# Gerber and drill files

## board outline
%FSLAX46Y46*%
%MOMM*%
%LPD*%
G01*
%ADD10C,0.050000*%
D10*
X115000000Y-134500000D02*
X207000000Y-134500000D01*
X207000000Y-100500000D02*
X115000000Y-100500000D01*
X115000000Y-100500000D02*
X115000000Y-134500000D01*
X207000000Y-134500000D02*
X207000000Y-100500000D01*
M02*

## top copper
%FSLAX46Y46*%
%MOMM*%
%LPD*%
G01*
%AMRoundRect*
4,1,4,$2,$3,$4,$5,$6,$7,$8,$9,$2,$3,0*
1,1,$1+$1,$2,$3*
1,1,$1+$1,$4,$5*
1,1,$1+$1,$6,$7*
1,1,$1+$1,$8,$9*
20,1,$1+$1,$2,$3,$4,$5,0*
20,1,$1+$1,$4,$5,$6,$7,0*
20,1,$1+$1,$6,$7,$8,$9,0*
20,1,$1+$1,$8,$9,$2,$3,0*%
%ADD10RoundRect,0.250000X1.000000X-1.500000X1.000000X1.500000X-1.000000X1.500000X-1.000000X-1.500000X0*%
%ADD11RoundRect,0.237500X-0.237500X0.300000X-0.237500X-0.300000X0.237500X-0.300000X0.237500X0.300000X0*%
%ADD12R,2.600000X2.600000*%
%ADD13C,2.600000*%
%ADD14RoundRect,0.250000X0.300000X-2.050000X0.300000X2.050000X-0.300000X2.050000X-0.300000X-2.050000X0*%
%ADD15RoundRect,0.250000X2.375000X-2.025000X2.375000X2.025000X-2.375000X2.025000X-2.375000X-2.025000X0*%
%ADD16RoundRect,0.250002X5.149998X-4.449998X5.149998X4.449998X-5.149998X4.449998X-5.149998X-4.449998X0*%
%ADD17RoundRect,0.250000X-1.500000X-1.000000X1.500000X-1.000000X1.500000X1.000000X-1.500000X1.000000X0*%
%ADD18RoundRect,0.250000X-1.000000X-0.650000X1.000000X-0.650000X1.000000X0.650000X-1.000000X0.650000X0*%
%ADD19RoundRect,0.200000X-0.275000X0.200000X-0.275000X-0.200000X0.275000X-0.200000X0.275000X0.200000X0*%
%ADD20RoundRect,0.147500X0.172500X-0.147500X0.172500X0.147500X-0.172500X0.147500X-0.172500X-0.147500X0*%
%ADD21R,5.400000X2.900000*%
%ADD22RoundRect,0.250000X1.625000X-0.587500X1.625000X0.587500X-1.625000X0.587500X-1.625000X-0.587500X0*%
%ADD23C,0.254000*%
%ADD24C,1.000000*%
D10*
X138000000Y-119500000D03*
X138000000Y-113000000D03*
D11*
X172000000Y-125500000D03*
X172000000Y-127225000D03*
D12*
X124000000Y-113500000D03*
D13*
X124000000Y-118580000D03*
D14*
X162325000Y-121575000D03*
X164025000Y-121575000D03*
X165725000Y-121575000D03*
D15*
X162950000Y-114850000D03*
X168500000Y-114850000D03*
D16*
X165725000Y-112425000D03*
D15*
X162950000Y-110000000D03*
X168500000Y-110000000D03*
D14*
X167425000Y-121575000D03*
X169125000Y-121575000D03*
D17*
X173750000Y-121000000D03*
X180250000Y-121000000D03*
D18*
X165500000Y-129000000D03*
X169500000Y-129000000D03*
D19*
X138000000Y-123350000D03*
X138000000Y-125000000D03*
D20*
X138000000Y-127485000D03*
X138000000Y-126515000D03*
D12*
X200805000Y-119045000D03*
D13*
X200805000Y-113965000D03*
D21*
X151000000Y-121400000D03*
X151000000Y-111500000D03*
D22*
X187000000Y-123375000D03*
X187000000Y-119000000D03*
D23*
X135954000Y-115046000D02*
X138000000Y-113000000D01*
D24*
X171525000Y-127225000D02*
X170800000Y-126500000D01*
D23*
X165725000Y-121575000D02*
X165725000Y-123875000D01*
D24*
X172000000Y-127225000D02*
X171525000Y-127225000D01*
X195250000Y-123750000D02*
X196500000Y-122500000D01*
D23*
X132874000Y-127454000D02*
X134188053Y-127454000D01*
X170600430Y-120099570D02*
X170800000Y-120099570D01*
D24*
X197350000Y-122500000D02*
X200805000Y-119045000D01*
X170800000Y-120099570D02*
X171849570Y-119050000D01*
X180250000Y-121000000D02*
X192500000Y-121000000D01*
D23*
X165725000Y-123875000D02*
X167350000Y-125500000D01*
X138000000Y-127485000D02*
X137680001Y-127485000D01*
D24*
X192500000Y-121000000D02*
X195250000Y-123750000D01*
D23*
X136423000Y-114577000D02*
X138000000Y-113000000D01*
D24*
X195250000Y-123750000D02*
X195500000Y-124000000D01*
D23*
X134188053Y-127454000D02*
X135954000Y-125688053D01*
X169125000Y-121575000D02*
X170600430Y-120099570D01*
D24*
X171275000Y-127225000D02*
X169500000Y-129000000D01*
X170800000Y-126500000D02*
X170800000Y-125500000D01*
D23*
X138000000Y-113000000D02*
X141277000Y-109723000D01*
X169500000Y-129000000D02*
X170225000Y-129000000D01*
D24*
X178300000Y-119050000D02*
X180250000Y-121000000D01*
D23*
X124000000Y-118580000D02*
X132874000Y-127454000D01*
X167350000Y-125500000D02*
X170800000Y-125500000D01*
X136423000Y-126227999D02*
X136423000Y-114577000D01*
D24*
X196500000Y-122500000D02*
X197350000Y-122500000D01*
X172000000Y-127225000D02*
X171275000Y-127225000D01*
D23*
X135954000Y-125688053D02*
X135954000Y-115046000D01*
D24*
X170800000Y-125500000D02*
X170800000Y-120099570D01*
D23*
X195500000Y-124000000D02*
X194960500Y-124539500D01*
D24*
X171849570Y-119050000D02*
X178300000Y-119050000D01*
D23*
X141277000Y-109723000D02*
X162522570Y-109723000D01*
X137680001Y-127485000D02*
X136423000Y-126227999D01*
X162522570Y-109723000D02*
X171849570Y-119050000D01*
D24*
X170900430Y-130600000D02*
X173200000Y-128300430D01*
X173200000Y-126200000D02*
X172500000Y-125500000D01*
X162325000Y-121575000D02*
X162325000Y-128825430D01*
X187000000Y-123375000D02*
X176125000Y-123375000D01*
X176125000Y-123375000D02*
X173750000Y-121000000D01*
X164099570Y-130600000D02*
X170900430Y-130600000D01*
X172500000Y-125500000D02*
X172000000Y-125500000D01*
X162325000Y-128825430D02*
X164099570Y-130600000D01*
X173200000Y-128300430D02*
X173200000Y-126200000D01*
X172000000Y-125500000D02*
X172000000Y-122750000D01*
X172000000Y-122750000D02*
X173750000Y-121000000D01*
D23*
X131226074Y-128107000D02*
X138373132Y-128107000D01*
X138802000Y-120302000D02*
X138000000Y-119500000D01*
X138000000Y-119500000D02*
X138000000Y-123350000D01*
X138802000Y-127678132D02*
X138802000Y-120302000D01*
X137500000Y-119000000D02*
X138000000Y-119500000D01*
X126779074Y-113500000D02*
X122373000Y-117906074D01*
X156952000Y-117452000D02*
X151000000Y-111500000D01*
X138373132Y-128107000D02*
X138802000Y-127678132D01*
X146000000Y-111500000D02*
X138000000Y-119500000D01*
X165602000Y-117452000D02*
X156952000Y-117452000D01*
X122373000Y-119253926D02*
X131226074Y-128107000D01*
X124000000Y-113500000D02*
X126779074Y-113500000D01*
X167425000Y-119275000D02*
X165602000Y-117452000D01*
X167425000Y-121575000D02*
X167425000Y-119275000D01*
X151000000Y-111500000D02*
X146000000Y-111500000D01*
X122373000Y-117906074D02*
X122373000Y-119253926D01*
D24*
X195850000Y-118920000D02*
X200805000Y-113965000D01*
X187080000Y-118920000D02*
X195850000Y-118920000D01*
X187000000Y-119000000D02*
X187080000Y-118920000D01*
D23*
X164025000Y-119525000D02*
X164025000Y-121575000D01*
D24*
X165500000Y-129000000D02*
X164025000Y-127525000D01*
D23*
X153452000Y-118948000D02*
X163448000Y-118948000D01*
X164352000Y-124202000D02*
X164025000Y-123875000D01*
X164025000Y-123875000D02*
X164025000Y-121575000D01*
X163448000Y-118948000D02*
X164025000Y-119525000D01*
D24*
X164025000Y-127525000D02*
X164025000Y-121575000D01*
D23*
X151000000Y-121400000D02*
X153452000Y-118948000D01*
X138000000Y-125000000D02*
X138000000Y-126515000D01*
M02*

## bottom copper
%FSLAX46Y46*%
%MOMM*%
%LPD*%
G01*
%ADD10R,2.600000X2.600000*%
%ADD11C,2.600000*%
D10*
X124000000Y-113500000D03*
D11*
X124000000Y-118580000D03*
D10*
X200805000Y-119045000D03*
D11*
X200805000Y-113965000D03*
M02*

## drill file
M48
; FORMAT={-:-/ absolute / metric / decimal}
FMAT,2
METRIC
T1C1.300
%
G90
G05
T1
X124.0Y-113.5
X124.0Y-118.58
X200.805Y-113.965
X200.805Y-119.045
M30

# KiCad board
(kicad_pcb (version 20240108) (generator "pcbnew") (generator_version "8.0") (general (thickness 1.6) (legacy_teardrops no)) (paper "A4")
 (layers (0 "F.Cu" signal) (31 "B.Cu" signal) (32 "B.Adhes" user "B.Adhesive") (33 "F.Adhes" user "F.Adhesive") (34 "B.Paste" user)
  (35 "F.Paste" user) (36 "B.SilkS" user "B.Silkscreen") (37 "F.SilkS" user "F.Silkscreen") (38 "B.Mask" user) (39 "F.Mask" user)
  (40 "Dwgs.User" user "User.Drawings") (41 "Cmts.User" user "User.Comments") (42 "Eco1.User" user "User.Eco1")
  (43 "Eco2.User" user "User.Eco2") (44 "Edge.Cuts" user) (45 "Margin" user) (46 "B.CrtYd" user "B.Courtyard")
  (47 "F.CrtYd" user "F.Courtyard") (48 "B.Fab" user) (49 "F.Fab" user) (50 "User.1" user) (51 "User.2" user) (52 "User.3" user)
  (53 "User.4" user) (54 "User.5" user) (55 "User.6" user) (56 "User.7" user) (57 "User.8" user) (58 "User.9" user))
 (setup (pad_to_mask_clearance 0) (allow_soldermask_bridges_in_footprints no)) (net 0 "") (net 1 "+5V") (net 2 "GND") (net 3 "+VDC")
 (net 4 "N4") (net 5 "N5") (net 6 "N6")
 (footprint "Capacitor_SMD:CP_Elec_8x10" (layer "F.Cu") (at 138 116.25 90)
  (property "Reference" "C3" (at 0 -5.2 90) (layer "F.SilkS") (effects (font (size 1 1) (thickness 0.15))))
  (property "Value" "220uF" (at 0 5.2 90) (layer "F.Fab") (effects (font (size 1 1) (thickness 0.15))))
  (pad "1" smd roundrect (at -3.25 0 90) (size 3.5 2.5) (layers "F.Cu" "F.Paste" "F.Mask") (roundrect_rratio 0.1) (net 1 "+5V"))
  (pad "2" smd roundrect (at 3.25 0 90) (size 3.5 2.5) (layers "F.Cu" "F.Paste" "F.Mask") (roundrect_rratio 0.1) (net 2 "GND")))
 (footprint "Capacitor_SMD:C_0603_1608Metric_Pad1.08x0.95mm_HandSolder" (layer "F.Cu") (at 172 126.3625 -90)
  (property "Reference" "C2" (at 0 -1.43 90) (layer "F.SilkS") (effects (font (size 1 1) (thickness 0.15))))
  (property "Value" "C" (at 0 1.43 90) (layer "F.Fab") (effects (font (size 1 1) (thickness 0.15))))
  (pad "1" smd roundrect (at -0.8625 0 270) (size 1.075 0.95) (layers "F.Cu" "F.Paste" "F.Mask") (roundrect_rratio 0.25) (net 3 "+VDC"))
  (pad "2" smd roundrect (at 0.8625 0 270) (size 1.075 0.95) (layers "F.Cu" "F.Paste" "F.Mask") (roundrect_rratio 0.25) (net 2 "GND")))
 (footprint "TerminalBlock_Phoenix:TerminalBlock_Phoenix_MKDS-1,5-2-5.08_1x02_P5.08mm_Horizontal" (layer "F.Cu") (at 124 113.5 -90)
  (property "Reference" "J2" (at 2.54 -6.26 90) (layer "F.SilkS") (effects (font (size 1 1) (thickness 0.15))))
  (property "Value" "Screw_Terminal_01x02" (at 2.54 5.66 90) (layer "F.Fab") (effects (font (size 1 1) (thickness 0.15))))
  (pad "1" thru_hole rect (at 0 0 270) (size 2.6 2.6) (drill 1.3) (layers "*.Cu" "*.Mask") (remove_unused_layers no) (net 1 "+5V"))
  (pad "2" thru_hole circle (at 5.08 0 270) (size 2.6 2.6) (drill 1.3) (layers "*.Cu" "*.Mask") (remove_unused_layers no) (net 2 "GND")))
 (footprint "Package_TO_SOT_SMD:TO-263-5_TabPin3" (layer "F.Cu") (at 165.725 113.925 90)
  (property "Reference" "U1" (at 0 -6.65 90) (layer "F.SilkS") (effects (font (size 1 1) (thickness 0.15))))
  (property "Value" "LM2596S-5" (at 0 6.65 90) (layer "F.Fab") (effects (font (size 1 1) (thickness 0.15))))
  (pad "1" smd roundrect (at -7.65 -3.4 90) (size 4.6 1.1) (layers "F.Cu" "F.Paste" "F.Mask") (roundrect_rratio 0.227273) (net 3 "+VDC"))
  (pad "2" smd roundrect (at -7.65 -1.7 90) (size 4.6 1.1) (layers "F.Cu" "F.Paste" "F.Mask") (roundrect_rratio 0.227273) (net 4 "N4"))
  (pad "3" smd roundrect (at -7.65 0 90) (size 4.6 1.1) (layers "F.Cu" "F.Paste" "F.Mask") (roundrect_rratio 0.227273) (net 2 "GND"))
  (pad "3" smd roundrect (at -0.925 -2.775 90) (size 4.55 5.25) (layers "F.Cu" "F.Paste") (roundrect_rratio 0.054945) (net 2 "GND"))
  (pad "3" smd roundrect (at -0.925 2.775 90) (size 4.55 5.25) (layers "F.Cu" "F.Paste") (roundrect_rratio 0.054945) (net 2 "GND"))
  (pad "3" smd roundrect (at 1.5 0 90) (size 9.4 10.8) (layers "F.Cu" "F.Mask") (roundrect_rratio 0.026596) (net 2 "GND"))
  (pad "3" smd roundrect (at 3.925 -2.775 90) (size 4.55 5.25) (layers "F.Cu" "F.Paste") (roundrect_rratio 0.054945) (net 2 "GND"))
  (pad "3" smd roundrect (at 3.925 2.775 90) (size 4.55 5.25) (layers "F.Cu" "F.Paste") (roundrect_rratio 0.054945) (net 2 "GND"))
  (pad "4" smd roundrect (at -7.65 1.7 90) (size 4.6 1.1) (layers "F.Cu" "F.Paste" "F.Mask") (roundrect_rratio 0.227273) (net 1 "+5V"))
  (pad "5" smd roundrect (at -7.65 3.4 90) (size 4.6 1.1) (layers "F.Cu" "F.Paste" "F.Mask") (roundrect_rratio 0.227273) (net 2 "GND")))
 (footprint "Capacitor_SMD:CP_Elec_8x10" (layer "F.Cu") (at 177 121)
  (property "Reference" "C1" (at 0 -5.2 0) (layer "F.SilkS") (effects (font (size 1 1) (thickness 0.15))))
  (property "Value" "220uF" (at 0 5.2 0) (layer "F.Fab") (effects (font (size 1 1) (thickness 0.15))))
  (pad "1" smd roundrect (at -3.25 0) (size 3.5 2.5) (layers "F.Cu" "F.Paste" "F.Mask") (roundrect_rratio 0.1) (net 3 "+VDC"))
  (pad "2" smd roundrect (at 3.25 0) (size 3.5 2.5) (layers "F.Cu" "F.Paste" "F.Mask") (roundrect_rratio 0.1) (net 2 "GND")))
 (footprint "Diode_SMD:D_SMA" (layer "F.Cu") (at 167.5 129)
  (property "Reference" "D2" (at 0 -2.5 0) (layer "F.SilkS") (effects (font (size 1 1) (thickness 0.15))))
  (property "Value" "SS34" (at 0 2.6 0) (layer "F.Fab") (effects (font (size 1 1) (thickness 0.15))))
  (pad "1" smd roundrect (at -2 0) (size 2.5 1.8) (layers "F.Cu" "F.Paste" "F.Mask") (roundrect_rratio 0.1388888889) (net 4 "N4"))
  (pad "2" smd roundrect (at 2 0) (size 2.5 1.8) (layers "F.Cu" "F.Paste" "F.Mask") (roundrect_rratio 0.1388888889) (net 2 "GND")))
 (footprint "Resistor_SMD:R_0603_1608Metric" (layer "F.Cu") (at 138 124.175 -90)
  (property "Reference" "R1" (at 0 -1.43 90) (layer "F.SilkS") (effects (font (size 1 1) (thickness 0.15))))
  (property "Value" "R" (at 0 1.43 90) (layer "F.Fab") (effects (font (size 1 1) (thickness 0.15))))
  (pad "1" smd roundrect (at -0.825 0 270) (size 0.8 0.95) (layers "F.Cu" "F.Paste" "F.Mask") (roundrect_rratio 0.25) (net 1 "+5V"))
  (pad "2" smd roundrect (at 0.825 0 270) (size 0.8 0.95) (layers "F.Cu" "F.Paste" "F.Mask") (roundrect_rratio 0.25) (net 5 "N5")))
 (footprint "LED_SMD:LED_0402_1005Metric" (layer "F.Cu") (at 138 127 90)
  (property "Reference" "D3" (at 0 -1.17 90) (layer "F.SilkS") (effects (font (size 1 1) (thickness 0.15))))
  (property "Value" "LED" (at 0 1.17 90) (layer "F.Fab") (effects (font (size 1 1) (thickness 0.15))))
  (pad "1" smd roundrect (at -0.485 0 90) (size 0.59 0.64) (layers "F.Cu" "F.Paste" "F.Mask") (roundrect_rratio 0.25) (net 2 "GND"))
  (pad "2" smd roundrect (at 0.485 0 90) (size 0.59 0.64) (layers "F.Cu" "F.Paste" "F.Mask") (roundrect_rratio 0.25) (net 5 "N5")))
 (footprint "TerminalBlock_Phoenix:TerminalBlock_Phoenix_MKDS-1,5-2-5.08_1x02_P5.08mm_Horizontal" (layer "F.Cu") (at 200.805 119.045 90)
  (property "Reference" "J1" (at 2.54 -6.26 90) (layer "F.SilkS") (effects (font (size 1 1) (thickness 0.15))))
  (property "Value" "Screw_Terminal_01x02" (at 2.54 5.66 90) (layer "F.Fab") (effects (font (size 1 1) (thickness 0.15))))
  (pad "1" thru_hole rect (at 0 0 90) (size 2.6 2.6) (drill 1.3) (layers "*.Cu" "*.Mask") (remove_unused_layers no) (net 2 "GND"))
  (pad "2" thru_hole circle (at 5.08 0 90) (size 2.6 2.6) (drill 1.3) (layers "*.Cu" "*.Mask") (remove_unused_layers no) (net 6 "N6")))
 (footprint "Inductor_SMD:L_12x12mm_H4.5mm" (layer "F.Cu") (at 151 116.45 90)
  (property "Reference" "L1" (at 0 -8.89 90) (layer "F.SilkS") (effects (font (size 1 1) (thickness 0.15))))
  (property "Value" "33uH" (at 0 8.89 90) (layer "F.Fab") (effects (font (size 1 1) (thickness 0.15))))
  (pad "1" smd rect (at -4.95 0 90) (size 2.9 5.4) (layers "F.Cu" "F.Paste" "F.Mask") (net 4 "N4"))
  (pad "2" smd rect (at 4.95 0 90) (size 2.9 5.4) (layers "F.Cu" "F.Paste" "F.Mask") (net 1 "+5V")))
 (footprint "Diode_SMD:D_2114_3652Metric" (layer "F.Cu") (at 187 121.1875 90)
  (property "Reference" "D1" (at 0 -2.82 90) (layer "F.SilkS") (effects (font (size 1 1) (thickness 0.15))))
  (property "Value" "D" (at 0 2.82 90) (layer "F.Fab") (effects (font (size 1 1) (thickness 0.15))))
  (pad "1" smd roundrect (at -2.1875 0 90) (size 1.675 3.75) (layers "F.Cu" "F.Paste" "F.Mask") (roundrect_rratio 0.149254) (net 3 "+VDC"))
  (pad "2" smd roundrect (at 2.1875 0 90) (size 1.675 3.75) (layers "F.Cu" "F.Paste" "F.Mask") (roundrect_rratio 0.149254) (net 6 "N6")))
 (gr_line (start 115 134.5) (end 207 134.5) (stroke (width 0.05) (type default)) (layer "Edge.Cuts"))
 (gr_line (start 207 100.5) (end 115 100.5) (stroke (width 0.05) (type default)) (layer "Edge.Cuts"))
 (gr_line (start 115 100.5) (end 115 134.5) (stroke (width 0.05) (type default)) (layer "Edge.Cuts"))
 (gr_line (start 207 134.5) (end 207 100.5) (stroke (width 0.05) (type default)) (layer "Edge.Cuts"))
 (segment (start 135.954 115.046) (end 138 113) (width 0.254) (layer "F.Cu") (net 2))
 (segment (start 171.525 127.225) (end 170.8 126.5) (width 1) (layer "F.Cu") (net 2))
 (segment (start 165.725 121.575) (end 165.725 123.875) (width 0.254) (layer "F.Cu") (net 2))
 (segment (start 172 127.225) (end 171.525 127.225) (width 1) (layer "F.Cu") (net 2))
 (segment (start 195.25 123.75) (end 196.5 122.5) (width 1) (layer "F.Cu") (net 2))
 (segment (start 132.874 127.454) (end 134.188053 127.454) (width 0.254) (layer "F.Cu") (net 2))
 (segment (start 170.60043 120.09957) (end 170.8 120.09957) (width 0.254) (layer "F.Cu") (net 2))
 (segment (start 197.35 122.5) (end 200.805 119.045) (width 1) (layer "F.Cu") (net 2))
 (segment (start 170.8 120.09957) (end 171.84957 119.05) (width 1) (layer "F.Cu") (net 2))
 (segment (start 180.25 121) (end 192.5 121) (width 1) (layer "F.Cu") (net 2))
 (segment (start 165.725 123.875) (end 167.35 125.5) (width 0.254) (layer "F.Cu") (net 2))
 (segment (start 138 127.485) (end 137.680001 127.485) (width 0.254) (layer "F.Cu") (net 2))
 (segment (start 192.5 121) (end 195.25 123.75) (width 1) (layer "F.Cu") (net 2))
 (segment (start 136.423 114.577) (end 138 113) (width 0.254) (layer "F.Cu") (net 2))
 (segment (start 195.25 123.75) (end 195.5 124) (width 1) (layer "F.Cu") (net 2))
 (segment (start 134.188053 127.454) (end 135.954 125.688053) (width 0.254) (layer "F.Cu") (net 2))
 (segment (start 169.125 121.575) (end 170.60043 120.09957) (width 0.254) (layer "F.Cu") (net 2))
 (segment (start 171.275 127.225) (end 169.5 129) (width 1) (layer "F.Cu") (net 2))
 (segment (start 170.8 126.5) (end 170.8 125.5) (width 1) (layer "F.Cu") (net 2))
 (segment (start 138 113) (end 141.277 109.723) (width 0.254) (layer "F.Cu") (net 2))
 (segment (start 169.5 129) (end 170.225 129) (width 0.254) (layer "F.Cu") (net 2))
 (segment (start 178.3 119.05) (end 180.25 121) (width 1) (layer "F.Cu") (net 2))
 (segment (start 124 118.58) (end 132.874 127.454) (width 0.254) (layer "F.Cu") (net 2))
 (segment (start 167.35 125.5) (end 170.8 125.5) (width 0.254) (layer "F.Cu") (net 2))
 (segment (start 136.423 126.227999) (end 136.423 114.577) (width 0.254) (layer "F.Cu") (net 2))
 (segment (start 196.5 122.5) (end 197.35 122.5) (width 1) (layer "F.Cu") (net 2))
 (segment (start 172 127.225) (end 171.275 127.225) (width 1) (layer "F.Cu") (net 2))
 (segment (start 135.954 125.688053) (end 135.954 115.046) (width 0.254) (layer "F.Cu") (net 2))
 (segment (start 170.8 125.5) (end 170.8 120.09957) (width 1) (layer "F.Cu") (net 2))
 (segment (start 195.5 124) (end 194.9605 124.5395) (width 0.254) (layer "F.Cu") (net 2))
 (segment (start 171.84957 119.05) (end 178.3 119.05) (width 1) (layer "F.Cu") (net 2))
 (segment (start 141.277 109.723) (end 162.52257 109.723) (width 0.254) (layer "F.Cu") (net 2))
 (segment (start 137.680001 127.485) (end 136.423 126.227999) (width 0.254) (layer "F.Cu") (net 2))
 (segment (start 162.52257 109.723) (end 171.84957 119.05) (width 0.254) (layer "F.Cu") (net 2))
 (segment (start 170.90043 130.6) (end 173.2 128.30043) (width 1) (layer "F.Cu") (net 3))
 (segment (start 173.2 126.2) (end 172.5 125.5) (width 1) (layer "F.Cu") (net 3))
 (segment (start 162.325 121.575) (end 162.325 128.82543) (width 1) (layer "F.Cu") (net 3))
 (segment (start 187 123.375) (end 176.125 123.375) (width 1) (layer "F.Cu") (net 3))
 (segment (start 176.125 123.375) (end 173.75 121) (width 1) (layer "F.Cu") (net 3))
 (segment (start 164.09957 130.6) (end 170.90043 130.6) (width 1) (layer "F.Cu") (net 3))
 (segment (start 172.5 125.5) (end 172 125.5) (width 1) (layer "F.Cu") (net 3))
 (segment (start 162.325 128.82543) (end 164.09957 130.6) (width 1) (layer "F.Cu") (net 3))
 (segment (start 173.2 128.30043) (end 173.2 126.2) (width 1) (layer "F.Cu") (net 3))
 (segment (start 172 125.5) (end 172 122.75) (width 1) (layer "F.Cu") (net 3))
 (segment (start 172 122.75) (end 173.75 121) (width 1) (layer "F.Cu") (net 3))
 (segment (start 131.226074 128.107) (end 138.373132 128.107) (width 0.254) (layer "F.Cu") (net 1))
 (segment (start 138.802 120.302) (end 138 119.5) (width 0.254) (layer "F.Cu") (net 1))
 (segment (start 138 119.5) (end 138 123.35) (width 0.254) (layer "F.Cu") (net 1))
 (segment (start 138.802 127.678132) (end 138.802 120.302) (width 0.254) (layer "F.Cu") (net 1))
 (segment (start 137.5 119) (end 138 119.5) (width 0.254) (layer "F.Cu") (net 1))
 (segment (start 126.779074 113.5) (end 122.373 117.906074) (width 0.254) (layer "F.Cu") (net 1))
 (segment (start 156.952 117.452) (end 151 111.5) (width 0.254) (layer "F.Cu") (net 1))
 (segment (start 138.373132 128.107) (end 138.802 127.678132) (width 0.254) (layer "F.Cu") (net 1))
 (segment (start 146 111.5) (end 138 119.5) (width 0.254) (layer "F.Cu") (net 1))
 (segment (start 165.602 117.452) (end 156.952 117.452) (width 0.254) (layer "F.Cu") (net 1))
 (segment (start 122.373 119.253926) (end 131.226074 128.107) (width 0.254) (layer "F.Cu") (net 1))
 (segment (start 124 113.5) (end 126.779074 113.5) (width 0.254) (layer "F.Cu") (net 1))
 (segment (start 167.425 119.275) (end 165.602 117.452) (width 0.254) (layer "F.Cu") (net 1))
 (segment (start 167.425 121.575) (end 167.425 119.275) (width 0.254) (layer "F.Cu") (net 1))
 (segment (start 151 111.5) (end 146 111.5) (width 0.254) (layer "F.Cu") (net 1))
 (segment (start 122.373 117.906074) (end 122.373 119.253926) (width 0.254) (layer "F.Cu") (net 1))
 (segment (start 195.85 118.92) (end 200.805 113.965) (width 1) (layer "F.Cu") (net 6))
 (segment (start 187.08 118.92) (end 195.85 118.92) (width 1) (layer "F.Cu") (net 6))
 (segment (start 187 119) (end 187.08 118.92) (width 1) (layer "F.Cu") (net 6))
 (segment (start 164.025 119.525) (end 164.025 121.575) (width 0.254) (layer "F.Cu") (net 4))
 (segment (start 165.5 129) (end 164.025 127.525) (width 1) (layer "F.Cu") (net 4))
 (segment (start 153.452 118.948) (end 163.448 118.948) (width 0.254) (layer "F.Cu") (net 4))
 (segment (start 164.352 124.202) (end 164.025 123.875) (width 0.254) (layer "F.Cu") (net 4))
 (segment (start 164.025 123.875) (end 164.025 121.575) (width 0.254) (layer "F.Cu") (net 4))
 (segment (start 163.448 118.948) (end 164.025 119.525) (width 0.254) (layer "F.Cu") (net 4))
 (segment (start 164.025 127.525) (end 164.025 121.575) (width 1) (layer "F.Cu") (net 4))
 (segment (start 151 121.4) (end 153.452 118.948) (width 0.254) (layer "F.Cu") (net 4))
 (segment (start 138 125) (end 138 126.515) (width 0.254) (layer "F.Cu") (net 5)))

